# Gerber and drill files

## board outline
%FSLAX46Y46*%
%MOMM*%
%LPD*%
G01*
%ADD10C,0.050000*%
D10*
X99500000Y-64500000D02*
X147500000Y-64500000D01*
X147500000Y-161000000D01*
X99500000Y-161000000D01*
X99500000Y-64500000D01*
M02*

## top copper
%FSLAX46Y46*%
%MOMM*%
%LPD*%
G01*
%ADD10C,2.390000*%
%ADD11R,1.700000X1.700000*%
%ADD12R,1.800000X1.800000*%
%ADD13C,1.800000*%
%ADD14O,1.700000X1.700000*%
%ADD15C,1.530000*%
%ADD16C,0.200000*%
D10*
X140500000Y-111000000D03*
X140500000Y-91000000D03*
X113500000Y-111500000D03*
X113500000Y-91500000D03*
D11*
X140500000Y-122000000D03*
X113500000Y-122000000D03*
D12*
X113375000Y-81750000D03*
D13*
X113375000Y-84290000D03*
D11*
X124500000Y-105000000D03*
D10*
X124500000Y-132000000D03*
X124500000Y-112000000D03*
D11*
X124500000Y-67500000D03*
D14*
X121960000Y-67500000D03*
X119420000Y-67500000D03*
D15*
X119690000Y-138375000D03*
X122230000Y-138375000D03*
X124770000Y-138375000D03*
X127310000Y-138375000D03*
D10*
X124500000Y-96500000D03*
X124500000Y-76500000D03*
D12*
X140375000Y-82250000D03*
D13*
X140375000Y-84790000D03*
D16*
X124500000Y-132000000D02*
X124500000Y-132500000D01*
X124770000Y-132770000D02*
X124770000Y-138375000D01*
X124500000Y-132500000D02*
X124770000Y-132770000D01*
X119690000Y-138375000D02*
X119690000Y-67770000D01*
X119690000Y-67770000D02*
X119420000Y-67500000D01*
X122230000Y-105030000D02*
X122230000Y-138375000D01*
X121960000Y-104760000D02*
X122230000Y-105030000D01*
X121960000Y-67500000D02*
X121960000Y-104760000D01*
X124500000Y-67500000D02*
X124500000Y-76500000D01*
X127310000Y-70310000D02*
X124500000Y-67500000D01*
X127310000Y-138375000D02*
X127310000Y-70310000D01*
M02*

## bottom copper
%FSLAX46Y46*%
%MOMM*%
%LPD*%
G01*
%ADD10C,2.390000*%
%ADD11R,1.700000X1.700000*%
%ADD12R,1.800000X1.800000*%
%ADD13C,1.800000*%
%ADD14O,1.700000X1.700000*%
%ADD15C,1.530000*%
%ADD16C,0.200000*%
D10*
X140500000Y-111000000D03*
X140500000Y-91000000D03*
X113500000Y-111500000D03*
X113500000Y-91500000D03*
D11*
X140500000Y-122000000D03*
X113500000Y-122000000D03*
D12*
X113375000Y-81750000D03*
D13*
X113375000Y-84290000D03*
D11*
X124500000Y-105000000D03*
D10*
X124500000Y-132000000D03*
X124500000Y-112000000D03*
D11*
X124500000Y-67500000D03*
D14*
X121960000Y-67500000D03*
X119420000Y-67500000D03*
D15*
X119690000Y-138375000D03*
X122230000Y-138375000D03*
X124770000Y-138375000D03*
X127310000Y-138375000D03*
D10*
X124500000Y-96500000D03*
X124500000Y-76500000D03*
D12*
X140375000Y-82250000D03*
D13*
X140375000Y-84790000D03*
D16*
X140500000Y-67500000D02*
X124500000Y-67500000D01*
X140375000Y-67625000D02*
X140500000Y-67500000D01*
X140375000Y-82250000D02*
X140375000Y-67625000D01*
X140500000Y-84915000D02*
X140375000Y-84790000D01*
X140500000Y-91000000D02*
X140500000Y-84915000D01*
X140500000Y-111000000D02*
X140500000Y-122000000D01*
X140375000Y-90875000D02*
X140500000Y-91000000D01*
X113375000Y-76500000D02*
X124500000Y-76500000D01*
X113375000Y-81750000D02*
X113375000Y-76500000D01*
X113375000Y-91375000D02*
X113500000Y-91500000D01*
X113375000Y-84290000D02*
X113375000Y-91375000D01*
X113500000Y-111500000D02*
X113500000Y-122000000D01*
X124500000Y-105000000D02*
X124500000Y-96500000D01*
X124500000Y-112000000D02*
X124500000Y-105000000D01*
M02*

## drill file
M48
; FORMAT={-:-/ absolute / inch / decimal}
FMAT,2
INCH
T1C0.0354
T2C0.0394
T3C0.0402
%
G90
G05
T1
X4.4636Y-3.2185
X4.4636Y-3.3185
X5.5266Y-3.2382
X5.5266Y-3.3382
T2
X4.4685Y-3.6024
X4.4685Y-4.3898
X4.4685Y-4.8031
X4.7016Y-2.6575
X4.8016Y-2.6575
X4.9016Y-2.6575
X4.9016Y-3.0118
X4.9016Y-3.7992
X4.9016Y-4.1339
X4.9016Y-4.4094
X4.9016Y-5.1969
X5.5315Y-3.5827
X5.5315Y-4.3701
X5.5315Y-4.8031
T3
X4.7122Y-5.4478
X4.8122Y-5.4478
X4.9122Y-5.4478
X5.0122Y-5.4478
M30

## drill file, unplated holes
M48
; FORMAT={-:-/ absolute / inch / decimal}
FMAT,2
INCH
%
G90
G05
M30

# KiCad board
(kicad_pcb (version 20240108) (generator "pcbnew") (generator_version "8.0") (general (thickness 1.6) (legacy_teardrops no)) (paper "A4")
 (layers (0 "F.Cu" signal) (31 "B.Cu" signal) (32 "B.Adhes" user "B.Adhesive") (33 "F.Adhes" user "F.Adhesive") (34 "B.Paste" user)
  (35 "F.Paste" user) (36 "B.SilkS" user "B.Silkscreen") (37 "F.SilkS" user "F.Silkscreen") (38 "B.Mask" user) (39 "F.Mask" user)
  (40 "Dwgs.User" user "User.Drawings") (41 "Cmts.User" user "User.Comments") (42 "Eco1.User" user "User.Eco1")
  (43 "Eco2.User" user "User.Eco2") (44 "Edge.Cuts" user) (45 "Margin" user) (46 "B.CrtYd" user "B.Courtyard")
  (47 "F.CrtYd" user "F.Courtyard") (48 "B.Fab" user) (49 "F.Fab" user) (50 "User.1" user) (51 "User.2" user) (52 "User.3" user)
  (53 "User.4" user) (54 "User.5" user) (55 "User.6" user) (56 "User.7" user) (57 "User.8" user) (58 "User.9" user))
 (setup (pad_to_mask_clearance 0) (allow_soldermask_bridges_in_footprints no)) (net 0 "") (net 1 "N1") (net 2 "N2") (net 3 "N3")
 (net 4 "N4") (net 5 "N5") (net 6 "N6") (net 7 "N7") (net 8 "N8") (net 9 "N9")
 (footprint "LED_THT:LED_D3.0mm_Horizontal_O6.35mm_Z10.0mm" (layer "F.Cu") (at 140.375 82.25 -90)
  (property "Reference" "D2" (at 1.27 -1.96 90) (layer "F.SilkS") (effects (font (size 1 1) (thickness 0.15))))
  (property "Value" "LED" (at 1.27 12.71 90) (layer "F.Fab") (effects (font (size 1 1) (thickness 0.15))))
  (pad "1" thru_hole rect (at 0 0 270) (size 1.8 1.8) (drill 0.9) (layers "*.Cu" "*.Mask") (remove_unused_layers no) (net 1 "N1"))
  (pad "2" thru_hole circle (at 2.54 0 270) (size 1.8 1.8) (drill 0.9) (layers "*.Cu" "*.Mask") (remove_unused_layers no) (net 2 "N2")))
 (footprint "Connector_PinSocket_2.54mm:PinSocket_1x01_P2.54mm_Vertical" (layer "F.Cu") (at 113.5 122)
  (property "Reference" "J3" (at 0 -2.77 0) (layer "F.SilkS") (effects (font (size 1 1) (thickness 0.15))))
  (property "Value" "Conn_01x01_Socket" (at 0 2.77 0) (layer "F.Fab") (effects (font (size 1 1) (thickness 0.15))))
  (pad "1" thru_hole rect (at 0 0) (size 1.7 1.7) (drill 1) (layers "*.Cu" "*.Mask") (remove_unused_layers no) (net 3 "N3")))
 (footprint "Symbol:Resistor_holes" (layer "F.Cu") (at 113.5 101.5 -90)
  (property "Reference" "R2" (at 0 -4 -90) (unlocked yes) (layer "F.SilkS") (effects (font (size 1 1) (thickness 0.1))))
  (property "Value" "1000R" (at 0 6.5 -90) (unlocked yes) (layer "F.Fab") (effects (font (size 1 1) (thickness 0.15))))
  (pad "1" thru_hole circle (at 10 0 270) (size 2.39 2.39) (drill 1) (layers "*.Cu" "*.Mask") (remove_unused_layers no) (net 3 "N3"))
  (pad "2" thru_hole circle (at -10 0 270) (size 2.39 2.39) (drill 1) (layers "*.Cu" "*.Mask") (remove_unused_layers no) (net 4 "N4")))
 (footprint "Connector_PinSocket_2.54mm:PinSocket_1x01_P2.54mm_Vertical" (layer "F.Cu") (at 140.5 122)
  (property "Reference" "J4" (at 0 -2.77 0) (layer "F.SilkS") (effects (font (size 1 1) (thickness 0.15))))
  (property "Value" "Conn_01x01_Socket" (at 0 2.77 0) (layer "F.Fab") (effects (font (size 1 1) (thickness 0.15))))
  (pad "1" thru_hole rect (at 0 0) (size 1.7 1.7) (drill 1) (layers "*.Cu" "*.Mask") (remove_unused_layers no) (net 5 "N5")))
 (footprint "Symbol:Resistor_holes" (layer "F.Cu") (at 140.5 101 -90)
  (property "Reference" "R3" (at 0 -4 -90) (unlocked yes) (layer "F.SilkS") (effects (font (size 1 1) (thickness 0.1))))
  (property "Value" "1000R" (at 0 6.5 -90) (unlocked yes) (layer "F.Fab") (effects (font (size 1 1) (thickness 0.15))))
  (pad "1" thru_hole circle (at 10 0 270) (size 2.39 2.39) (drill 1) (layers "*.Cu" "*.Mask") (remove_unused_layers no) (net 5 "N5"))
  (pad "2" thru_hole circle (at -10 0 270) (size 2.39 2.39) (drill 1) (layers "*.Cu" "*.Mask") (remove_unused_layers no) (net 2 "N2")))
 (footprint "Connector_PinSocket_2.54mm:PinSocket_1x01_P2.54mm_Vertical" (layer "F.Cu") (at 124.5 105)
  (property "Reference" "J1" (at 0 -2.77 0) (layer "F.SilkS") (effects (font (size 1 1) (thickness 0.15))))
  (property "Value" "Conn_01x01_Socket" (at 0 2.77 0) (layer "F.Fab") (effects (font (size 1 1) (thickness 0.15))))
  (pad "1" thru_hole rect (at 0 0) (size 1.7 1.7) (drill 1) (layers "*.Cu" "*.Mask") (remove_unused_layers no) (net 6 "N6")))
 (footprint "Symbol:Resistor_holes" (layer "F.Cu") (at 124.5 122 -90)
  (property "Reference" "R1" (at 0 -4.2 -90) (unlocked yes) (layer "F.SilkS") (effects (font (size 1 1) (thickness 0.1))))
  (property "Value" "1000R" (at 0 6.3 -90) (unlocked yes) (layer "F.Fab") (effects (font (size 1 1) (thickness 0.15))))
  (pad "1" thru_hole circle (at 10 0 270) (size 2.39 2.39) (drill 1) (layers "*.Cu" "*.Mask") (remove_unused_layers no) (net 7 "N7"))
  (pad "2" thru_hole circle (at -10 0 270) (size 2.39 2.39) (drill 1) (layers "*.Cu" "*.Mask") (remove_unused_layers no) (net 6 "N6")))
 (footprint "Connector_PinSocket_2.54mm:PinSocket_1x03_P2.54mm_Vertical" (layer "F.Cu") (at 124.5 67.5 -90)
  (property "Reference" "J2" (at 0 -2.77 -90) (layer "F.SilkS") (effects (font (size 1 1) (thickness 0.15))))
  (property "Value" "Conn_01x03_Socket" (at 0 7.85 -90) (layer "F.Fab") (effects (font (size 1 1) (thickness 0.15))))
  (pad "1" thru_hole rect (at 0 0 270) (size 1.7 1.7) (drill 1) (layers "*.Cu" "*.Mask") (remove_unused_layers no) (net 1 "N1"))
  (pad "2" thru_hole oval (at 0 2.54 270) (size 1.7 1.7) (drill 1) (layers "*.Cu" "*.Mask") (remove_unused_layers no) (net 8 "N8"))
  (pad "3" thru_hole oval (at 0 5.08 270) (size 1.7 1.7) (drill 1) (layers "*.Cu" "*.Mask") (remove_unused_layers no) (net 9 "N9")))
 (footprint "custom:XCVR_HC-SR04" (layer "F.Cu") (at 123.5 138.375)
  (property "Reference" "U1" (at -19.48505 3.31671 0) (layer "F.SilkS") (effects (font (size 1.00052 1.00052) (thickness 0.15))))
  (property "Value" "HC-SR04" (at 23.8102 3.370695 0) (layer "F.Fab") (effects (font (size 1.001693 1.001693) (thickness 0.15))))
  (pad "1" thru_hole circle (at -3.81 0) (size 1.53 1.53) (drill 1.02) (layers "*.Cu" "*.Mask") (remove_unused_layers no) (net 9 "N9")
   (solder_mask_margin 0.102))
  (pad "2" thru_hole circle (at -1.27 0) (size 1.53 1.53) (drill 1.02) (layers "*.Cu" "*.Mask") (remove_unused_layers no) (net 8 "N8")
   (solder_mask_margin 0.102))
  (pad "3" thru_hole circle (at 1.27 0) (size 1.53 1.53) (drill 1.02) (layers "*.Cu" "*.Mask") (remove_unused_layers no) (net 7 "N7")
   (solder_mask_margin 0.102))
  (pad "4" thru_hole circle (at 3.81 0) (size 1.53 1.53) (drill 1.02) (layers "*.Cu" "*.Mask") (remove_unused_layers no) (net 1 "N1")
   (solder_mask_margin 0.102)))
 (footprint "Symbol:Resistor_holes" (layer "F.Cu") (at 124.5 86.5 -90)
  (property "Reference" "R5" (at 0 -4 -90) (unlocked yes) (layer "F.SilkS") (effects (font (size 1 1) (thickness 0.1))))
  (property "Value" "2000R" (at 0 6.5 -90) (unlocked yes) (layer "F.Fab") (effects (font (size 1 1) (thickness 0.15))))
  (pad "1" thru_hole circle (at 10 0 270) (size 2.39 2.39) (drill 1) (layers "*.Cu" "*.Mask") (remove_unused_layers no) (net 6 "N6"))
  (pad "2" thru_hole circle (at -10 0 270) (size 2.39 2.39) (drill 1) (layers "*.Cu" "*.Mask") (remove_unused_layers no) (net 1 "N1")))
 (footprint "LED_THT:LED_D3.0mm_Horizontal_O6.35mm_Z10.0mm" (layer "F.Cu") (at 113.375 81.75 -90)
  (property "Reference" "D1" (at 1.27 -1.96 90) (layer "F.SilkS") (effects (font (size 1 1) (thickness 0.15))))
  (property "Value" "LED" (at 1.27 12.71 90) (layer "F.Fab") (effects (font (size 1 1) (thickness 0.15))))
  (pad "1" thru_hole rect (at 0 0 270) (size 1.8 1.8) (drill 0.9) (layers "*.Cu" "*.Mask") (remove_unused_layers no) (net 1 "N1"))
  (pad "2" thru_hole circle (at 2.54 0 270) (size 1.8 1.8) (drill 0.9) (layers "*.Cu" "*.Mask") (remove_unused_layers no) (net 4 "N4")))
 (gr_rect (start 99.5 64.5) (end 147.5 161) (stroke (width 0.05) (type default)) (fill none) (layer "Edge.Cuts"))
 (segment (start 124.5 105) (end 124.5 96.5) (width 0.2) (layer "B.Cu") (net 6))
 (segment (start 124.5 112) (end 124.5 105) (width 0.2) (layer "B.Cu") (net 6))
 (segment (start 124.5 132) (end 124.5 132.5) (width 0.2) (layer "F.Cu") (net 7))
 (segment (start 124.77 132.77) (end 124.77 138.375) (width 0.2) (layer "F.Cu") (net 7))
 (segment (start 124.5 132.5) (end 124.77 132.77) (width 0.2) (layer "F.Cu") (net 7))
 (segment (start 119.69 138.375) (end 119.69 67.77) (width 0.2) (layer "F.Cu") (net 9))
 (segment (start 119.69 67.77) (end 119.42 67.5) (width 0.2) (layer "F.Cu") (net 9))
 (segment (start 122.23 105.03) (end 122.23 138.375) (width 0.2) (layer "F.Cu") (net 8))
 (segment (start 121.96 104.76) (end 122.23 105.03) (width 0.2) (layer "F.Cu") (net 8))
 (segment (start 121.96 67.5) (end 121.96 104.76) (width 0.2) (layer "F.Cu") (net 8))
 (segment (start 113.375 84.29) (end 113.375 91.375) (width 0.2) (layer "B.Cu") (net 4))
 (segment (start 113.375 91.375) (end 113.5 91.5) (width 0.2) (layer "B.Cu") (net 4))
 (segment (start 124.5 67.5) (end 124.5 76.5) (width 0.2) (layer "F.Cu") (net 1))
 (segment (start 127.31 70.31) (end 124.5 67.5) (width 0.2) (layer "F.Cu") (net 1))
 (segment (start 127.31 138.375) (end 127.31 70.31) (width 0.2) (layer "F.Cu") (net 1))
 (segment (start 140.375 82.25) (end 140.375 67.625) (width 0.2) (layer "B.Cu") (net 1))
 (segment (start 113.375 76.5) (end 124.5 76.5) (width 0.2) (layer "B.Cu") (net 1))
 (segment (start 113.375 81.75) (end 113.375 76.5) (width 0.2) (layer "B.Cu") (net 1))
 (segment (start 140.5 67.5) (end 124.5 67.5) (width 0.2) (layer "B.Cu") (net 1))
 (segment (start 140.375 67.625) (end 140.5 67.5) (width 0.2) (layer "B.Cu") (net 1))
 (segment (start 140.5 91) (end 140.5 84.915) (width 0.2) (layer "B.Cu") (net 2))
 (segment (start 140.5 84.915) (end 140.375 84.79) (width 0.2) (layer "B.Cu") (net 2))
 (segment (start 140.375 90.875) (end 140.5 91) (width 0.2) (layer "B.Cu") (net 2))
 (segment (start 113.5 111.5) (end 113.5 122) (width 0.2) (layer "B.Cu") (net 3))
 (segment (start 140.5 111) (end 140.5 122) (width 0.2) (layer "B.Cu") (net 5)))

